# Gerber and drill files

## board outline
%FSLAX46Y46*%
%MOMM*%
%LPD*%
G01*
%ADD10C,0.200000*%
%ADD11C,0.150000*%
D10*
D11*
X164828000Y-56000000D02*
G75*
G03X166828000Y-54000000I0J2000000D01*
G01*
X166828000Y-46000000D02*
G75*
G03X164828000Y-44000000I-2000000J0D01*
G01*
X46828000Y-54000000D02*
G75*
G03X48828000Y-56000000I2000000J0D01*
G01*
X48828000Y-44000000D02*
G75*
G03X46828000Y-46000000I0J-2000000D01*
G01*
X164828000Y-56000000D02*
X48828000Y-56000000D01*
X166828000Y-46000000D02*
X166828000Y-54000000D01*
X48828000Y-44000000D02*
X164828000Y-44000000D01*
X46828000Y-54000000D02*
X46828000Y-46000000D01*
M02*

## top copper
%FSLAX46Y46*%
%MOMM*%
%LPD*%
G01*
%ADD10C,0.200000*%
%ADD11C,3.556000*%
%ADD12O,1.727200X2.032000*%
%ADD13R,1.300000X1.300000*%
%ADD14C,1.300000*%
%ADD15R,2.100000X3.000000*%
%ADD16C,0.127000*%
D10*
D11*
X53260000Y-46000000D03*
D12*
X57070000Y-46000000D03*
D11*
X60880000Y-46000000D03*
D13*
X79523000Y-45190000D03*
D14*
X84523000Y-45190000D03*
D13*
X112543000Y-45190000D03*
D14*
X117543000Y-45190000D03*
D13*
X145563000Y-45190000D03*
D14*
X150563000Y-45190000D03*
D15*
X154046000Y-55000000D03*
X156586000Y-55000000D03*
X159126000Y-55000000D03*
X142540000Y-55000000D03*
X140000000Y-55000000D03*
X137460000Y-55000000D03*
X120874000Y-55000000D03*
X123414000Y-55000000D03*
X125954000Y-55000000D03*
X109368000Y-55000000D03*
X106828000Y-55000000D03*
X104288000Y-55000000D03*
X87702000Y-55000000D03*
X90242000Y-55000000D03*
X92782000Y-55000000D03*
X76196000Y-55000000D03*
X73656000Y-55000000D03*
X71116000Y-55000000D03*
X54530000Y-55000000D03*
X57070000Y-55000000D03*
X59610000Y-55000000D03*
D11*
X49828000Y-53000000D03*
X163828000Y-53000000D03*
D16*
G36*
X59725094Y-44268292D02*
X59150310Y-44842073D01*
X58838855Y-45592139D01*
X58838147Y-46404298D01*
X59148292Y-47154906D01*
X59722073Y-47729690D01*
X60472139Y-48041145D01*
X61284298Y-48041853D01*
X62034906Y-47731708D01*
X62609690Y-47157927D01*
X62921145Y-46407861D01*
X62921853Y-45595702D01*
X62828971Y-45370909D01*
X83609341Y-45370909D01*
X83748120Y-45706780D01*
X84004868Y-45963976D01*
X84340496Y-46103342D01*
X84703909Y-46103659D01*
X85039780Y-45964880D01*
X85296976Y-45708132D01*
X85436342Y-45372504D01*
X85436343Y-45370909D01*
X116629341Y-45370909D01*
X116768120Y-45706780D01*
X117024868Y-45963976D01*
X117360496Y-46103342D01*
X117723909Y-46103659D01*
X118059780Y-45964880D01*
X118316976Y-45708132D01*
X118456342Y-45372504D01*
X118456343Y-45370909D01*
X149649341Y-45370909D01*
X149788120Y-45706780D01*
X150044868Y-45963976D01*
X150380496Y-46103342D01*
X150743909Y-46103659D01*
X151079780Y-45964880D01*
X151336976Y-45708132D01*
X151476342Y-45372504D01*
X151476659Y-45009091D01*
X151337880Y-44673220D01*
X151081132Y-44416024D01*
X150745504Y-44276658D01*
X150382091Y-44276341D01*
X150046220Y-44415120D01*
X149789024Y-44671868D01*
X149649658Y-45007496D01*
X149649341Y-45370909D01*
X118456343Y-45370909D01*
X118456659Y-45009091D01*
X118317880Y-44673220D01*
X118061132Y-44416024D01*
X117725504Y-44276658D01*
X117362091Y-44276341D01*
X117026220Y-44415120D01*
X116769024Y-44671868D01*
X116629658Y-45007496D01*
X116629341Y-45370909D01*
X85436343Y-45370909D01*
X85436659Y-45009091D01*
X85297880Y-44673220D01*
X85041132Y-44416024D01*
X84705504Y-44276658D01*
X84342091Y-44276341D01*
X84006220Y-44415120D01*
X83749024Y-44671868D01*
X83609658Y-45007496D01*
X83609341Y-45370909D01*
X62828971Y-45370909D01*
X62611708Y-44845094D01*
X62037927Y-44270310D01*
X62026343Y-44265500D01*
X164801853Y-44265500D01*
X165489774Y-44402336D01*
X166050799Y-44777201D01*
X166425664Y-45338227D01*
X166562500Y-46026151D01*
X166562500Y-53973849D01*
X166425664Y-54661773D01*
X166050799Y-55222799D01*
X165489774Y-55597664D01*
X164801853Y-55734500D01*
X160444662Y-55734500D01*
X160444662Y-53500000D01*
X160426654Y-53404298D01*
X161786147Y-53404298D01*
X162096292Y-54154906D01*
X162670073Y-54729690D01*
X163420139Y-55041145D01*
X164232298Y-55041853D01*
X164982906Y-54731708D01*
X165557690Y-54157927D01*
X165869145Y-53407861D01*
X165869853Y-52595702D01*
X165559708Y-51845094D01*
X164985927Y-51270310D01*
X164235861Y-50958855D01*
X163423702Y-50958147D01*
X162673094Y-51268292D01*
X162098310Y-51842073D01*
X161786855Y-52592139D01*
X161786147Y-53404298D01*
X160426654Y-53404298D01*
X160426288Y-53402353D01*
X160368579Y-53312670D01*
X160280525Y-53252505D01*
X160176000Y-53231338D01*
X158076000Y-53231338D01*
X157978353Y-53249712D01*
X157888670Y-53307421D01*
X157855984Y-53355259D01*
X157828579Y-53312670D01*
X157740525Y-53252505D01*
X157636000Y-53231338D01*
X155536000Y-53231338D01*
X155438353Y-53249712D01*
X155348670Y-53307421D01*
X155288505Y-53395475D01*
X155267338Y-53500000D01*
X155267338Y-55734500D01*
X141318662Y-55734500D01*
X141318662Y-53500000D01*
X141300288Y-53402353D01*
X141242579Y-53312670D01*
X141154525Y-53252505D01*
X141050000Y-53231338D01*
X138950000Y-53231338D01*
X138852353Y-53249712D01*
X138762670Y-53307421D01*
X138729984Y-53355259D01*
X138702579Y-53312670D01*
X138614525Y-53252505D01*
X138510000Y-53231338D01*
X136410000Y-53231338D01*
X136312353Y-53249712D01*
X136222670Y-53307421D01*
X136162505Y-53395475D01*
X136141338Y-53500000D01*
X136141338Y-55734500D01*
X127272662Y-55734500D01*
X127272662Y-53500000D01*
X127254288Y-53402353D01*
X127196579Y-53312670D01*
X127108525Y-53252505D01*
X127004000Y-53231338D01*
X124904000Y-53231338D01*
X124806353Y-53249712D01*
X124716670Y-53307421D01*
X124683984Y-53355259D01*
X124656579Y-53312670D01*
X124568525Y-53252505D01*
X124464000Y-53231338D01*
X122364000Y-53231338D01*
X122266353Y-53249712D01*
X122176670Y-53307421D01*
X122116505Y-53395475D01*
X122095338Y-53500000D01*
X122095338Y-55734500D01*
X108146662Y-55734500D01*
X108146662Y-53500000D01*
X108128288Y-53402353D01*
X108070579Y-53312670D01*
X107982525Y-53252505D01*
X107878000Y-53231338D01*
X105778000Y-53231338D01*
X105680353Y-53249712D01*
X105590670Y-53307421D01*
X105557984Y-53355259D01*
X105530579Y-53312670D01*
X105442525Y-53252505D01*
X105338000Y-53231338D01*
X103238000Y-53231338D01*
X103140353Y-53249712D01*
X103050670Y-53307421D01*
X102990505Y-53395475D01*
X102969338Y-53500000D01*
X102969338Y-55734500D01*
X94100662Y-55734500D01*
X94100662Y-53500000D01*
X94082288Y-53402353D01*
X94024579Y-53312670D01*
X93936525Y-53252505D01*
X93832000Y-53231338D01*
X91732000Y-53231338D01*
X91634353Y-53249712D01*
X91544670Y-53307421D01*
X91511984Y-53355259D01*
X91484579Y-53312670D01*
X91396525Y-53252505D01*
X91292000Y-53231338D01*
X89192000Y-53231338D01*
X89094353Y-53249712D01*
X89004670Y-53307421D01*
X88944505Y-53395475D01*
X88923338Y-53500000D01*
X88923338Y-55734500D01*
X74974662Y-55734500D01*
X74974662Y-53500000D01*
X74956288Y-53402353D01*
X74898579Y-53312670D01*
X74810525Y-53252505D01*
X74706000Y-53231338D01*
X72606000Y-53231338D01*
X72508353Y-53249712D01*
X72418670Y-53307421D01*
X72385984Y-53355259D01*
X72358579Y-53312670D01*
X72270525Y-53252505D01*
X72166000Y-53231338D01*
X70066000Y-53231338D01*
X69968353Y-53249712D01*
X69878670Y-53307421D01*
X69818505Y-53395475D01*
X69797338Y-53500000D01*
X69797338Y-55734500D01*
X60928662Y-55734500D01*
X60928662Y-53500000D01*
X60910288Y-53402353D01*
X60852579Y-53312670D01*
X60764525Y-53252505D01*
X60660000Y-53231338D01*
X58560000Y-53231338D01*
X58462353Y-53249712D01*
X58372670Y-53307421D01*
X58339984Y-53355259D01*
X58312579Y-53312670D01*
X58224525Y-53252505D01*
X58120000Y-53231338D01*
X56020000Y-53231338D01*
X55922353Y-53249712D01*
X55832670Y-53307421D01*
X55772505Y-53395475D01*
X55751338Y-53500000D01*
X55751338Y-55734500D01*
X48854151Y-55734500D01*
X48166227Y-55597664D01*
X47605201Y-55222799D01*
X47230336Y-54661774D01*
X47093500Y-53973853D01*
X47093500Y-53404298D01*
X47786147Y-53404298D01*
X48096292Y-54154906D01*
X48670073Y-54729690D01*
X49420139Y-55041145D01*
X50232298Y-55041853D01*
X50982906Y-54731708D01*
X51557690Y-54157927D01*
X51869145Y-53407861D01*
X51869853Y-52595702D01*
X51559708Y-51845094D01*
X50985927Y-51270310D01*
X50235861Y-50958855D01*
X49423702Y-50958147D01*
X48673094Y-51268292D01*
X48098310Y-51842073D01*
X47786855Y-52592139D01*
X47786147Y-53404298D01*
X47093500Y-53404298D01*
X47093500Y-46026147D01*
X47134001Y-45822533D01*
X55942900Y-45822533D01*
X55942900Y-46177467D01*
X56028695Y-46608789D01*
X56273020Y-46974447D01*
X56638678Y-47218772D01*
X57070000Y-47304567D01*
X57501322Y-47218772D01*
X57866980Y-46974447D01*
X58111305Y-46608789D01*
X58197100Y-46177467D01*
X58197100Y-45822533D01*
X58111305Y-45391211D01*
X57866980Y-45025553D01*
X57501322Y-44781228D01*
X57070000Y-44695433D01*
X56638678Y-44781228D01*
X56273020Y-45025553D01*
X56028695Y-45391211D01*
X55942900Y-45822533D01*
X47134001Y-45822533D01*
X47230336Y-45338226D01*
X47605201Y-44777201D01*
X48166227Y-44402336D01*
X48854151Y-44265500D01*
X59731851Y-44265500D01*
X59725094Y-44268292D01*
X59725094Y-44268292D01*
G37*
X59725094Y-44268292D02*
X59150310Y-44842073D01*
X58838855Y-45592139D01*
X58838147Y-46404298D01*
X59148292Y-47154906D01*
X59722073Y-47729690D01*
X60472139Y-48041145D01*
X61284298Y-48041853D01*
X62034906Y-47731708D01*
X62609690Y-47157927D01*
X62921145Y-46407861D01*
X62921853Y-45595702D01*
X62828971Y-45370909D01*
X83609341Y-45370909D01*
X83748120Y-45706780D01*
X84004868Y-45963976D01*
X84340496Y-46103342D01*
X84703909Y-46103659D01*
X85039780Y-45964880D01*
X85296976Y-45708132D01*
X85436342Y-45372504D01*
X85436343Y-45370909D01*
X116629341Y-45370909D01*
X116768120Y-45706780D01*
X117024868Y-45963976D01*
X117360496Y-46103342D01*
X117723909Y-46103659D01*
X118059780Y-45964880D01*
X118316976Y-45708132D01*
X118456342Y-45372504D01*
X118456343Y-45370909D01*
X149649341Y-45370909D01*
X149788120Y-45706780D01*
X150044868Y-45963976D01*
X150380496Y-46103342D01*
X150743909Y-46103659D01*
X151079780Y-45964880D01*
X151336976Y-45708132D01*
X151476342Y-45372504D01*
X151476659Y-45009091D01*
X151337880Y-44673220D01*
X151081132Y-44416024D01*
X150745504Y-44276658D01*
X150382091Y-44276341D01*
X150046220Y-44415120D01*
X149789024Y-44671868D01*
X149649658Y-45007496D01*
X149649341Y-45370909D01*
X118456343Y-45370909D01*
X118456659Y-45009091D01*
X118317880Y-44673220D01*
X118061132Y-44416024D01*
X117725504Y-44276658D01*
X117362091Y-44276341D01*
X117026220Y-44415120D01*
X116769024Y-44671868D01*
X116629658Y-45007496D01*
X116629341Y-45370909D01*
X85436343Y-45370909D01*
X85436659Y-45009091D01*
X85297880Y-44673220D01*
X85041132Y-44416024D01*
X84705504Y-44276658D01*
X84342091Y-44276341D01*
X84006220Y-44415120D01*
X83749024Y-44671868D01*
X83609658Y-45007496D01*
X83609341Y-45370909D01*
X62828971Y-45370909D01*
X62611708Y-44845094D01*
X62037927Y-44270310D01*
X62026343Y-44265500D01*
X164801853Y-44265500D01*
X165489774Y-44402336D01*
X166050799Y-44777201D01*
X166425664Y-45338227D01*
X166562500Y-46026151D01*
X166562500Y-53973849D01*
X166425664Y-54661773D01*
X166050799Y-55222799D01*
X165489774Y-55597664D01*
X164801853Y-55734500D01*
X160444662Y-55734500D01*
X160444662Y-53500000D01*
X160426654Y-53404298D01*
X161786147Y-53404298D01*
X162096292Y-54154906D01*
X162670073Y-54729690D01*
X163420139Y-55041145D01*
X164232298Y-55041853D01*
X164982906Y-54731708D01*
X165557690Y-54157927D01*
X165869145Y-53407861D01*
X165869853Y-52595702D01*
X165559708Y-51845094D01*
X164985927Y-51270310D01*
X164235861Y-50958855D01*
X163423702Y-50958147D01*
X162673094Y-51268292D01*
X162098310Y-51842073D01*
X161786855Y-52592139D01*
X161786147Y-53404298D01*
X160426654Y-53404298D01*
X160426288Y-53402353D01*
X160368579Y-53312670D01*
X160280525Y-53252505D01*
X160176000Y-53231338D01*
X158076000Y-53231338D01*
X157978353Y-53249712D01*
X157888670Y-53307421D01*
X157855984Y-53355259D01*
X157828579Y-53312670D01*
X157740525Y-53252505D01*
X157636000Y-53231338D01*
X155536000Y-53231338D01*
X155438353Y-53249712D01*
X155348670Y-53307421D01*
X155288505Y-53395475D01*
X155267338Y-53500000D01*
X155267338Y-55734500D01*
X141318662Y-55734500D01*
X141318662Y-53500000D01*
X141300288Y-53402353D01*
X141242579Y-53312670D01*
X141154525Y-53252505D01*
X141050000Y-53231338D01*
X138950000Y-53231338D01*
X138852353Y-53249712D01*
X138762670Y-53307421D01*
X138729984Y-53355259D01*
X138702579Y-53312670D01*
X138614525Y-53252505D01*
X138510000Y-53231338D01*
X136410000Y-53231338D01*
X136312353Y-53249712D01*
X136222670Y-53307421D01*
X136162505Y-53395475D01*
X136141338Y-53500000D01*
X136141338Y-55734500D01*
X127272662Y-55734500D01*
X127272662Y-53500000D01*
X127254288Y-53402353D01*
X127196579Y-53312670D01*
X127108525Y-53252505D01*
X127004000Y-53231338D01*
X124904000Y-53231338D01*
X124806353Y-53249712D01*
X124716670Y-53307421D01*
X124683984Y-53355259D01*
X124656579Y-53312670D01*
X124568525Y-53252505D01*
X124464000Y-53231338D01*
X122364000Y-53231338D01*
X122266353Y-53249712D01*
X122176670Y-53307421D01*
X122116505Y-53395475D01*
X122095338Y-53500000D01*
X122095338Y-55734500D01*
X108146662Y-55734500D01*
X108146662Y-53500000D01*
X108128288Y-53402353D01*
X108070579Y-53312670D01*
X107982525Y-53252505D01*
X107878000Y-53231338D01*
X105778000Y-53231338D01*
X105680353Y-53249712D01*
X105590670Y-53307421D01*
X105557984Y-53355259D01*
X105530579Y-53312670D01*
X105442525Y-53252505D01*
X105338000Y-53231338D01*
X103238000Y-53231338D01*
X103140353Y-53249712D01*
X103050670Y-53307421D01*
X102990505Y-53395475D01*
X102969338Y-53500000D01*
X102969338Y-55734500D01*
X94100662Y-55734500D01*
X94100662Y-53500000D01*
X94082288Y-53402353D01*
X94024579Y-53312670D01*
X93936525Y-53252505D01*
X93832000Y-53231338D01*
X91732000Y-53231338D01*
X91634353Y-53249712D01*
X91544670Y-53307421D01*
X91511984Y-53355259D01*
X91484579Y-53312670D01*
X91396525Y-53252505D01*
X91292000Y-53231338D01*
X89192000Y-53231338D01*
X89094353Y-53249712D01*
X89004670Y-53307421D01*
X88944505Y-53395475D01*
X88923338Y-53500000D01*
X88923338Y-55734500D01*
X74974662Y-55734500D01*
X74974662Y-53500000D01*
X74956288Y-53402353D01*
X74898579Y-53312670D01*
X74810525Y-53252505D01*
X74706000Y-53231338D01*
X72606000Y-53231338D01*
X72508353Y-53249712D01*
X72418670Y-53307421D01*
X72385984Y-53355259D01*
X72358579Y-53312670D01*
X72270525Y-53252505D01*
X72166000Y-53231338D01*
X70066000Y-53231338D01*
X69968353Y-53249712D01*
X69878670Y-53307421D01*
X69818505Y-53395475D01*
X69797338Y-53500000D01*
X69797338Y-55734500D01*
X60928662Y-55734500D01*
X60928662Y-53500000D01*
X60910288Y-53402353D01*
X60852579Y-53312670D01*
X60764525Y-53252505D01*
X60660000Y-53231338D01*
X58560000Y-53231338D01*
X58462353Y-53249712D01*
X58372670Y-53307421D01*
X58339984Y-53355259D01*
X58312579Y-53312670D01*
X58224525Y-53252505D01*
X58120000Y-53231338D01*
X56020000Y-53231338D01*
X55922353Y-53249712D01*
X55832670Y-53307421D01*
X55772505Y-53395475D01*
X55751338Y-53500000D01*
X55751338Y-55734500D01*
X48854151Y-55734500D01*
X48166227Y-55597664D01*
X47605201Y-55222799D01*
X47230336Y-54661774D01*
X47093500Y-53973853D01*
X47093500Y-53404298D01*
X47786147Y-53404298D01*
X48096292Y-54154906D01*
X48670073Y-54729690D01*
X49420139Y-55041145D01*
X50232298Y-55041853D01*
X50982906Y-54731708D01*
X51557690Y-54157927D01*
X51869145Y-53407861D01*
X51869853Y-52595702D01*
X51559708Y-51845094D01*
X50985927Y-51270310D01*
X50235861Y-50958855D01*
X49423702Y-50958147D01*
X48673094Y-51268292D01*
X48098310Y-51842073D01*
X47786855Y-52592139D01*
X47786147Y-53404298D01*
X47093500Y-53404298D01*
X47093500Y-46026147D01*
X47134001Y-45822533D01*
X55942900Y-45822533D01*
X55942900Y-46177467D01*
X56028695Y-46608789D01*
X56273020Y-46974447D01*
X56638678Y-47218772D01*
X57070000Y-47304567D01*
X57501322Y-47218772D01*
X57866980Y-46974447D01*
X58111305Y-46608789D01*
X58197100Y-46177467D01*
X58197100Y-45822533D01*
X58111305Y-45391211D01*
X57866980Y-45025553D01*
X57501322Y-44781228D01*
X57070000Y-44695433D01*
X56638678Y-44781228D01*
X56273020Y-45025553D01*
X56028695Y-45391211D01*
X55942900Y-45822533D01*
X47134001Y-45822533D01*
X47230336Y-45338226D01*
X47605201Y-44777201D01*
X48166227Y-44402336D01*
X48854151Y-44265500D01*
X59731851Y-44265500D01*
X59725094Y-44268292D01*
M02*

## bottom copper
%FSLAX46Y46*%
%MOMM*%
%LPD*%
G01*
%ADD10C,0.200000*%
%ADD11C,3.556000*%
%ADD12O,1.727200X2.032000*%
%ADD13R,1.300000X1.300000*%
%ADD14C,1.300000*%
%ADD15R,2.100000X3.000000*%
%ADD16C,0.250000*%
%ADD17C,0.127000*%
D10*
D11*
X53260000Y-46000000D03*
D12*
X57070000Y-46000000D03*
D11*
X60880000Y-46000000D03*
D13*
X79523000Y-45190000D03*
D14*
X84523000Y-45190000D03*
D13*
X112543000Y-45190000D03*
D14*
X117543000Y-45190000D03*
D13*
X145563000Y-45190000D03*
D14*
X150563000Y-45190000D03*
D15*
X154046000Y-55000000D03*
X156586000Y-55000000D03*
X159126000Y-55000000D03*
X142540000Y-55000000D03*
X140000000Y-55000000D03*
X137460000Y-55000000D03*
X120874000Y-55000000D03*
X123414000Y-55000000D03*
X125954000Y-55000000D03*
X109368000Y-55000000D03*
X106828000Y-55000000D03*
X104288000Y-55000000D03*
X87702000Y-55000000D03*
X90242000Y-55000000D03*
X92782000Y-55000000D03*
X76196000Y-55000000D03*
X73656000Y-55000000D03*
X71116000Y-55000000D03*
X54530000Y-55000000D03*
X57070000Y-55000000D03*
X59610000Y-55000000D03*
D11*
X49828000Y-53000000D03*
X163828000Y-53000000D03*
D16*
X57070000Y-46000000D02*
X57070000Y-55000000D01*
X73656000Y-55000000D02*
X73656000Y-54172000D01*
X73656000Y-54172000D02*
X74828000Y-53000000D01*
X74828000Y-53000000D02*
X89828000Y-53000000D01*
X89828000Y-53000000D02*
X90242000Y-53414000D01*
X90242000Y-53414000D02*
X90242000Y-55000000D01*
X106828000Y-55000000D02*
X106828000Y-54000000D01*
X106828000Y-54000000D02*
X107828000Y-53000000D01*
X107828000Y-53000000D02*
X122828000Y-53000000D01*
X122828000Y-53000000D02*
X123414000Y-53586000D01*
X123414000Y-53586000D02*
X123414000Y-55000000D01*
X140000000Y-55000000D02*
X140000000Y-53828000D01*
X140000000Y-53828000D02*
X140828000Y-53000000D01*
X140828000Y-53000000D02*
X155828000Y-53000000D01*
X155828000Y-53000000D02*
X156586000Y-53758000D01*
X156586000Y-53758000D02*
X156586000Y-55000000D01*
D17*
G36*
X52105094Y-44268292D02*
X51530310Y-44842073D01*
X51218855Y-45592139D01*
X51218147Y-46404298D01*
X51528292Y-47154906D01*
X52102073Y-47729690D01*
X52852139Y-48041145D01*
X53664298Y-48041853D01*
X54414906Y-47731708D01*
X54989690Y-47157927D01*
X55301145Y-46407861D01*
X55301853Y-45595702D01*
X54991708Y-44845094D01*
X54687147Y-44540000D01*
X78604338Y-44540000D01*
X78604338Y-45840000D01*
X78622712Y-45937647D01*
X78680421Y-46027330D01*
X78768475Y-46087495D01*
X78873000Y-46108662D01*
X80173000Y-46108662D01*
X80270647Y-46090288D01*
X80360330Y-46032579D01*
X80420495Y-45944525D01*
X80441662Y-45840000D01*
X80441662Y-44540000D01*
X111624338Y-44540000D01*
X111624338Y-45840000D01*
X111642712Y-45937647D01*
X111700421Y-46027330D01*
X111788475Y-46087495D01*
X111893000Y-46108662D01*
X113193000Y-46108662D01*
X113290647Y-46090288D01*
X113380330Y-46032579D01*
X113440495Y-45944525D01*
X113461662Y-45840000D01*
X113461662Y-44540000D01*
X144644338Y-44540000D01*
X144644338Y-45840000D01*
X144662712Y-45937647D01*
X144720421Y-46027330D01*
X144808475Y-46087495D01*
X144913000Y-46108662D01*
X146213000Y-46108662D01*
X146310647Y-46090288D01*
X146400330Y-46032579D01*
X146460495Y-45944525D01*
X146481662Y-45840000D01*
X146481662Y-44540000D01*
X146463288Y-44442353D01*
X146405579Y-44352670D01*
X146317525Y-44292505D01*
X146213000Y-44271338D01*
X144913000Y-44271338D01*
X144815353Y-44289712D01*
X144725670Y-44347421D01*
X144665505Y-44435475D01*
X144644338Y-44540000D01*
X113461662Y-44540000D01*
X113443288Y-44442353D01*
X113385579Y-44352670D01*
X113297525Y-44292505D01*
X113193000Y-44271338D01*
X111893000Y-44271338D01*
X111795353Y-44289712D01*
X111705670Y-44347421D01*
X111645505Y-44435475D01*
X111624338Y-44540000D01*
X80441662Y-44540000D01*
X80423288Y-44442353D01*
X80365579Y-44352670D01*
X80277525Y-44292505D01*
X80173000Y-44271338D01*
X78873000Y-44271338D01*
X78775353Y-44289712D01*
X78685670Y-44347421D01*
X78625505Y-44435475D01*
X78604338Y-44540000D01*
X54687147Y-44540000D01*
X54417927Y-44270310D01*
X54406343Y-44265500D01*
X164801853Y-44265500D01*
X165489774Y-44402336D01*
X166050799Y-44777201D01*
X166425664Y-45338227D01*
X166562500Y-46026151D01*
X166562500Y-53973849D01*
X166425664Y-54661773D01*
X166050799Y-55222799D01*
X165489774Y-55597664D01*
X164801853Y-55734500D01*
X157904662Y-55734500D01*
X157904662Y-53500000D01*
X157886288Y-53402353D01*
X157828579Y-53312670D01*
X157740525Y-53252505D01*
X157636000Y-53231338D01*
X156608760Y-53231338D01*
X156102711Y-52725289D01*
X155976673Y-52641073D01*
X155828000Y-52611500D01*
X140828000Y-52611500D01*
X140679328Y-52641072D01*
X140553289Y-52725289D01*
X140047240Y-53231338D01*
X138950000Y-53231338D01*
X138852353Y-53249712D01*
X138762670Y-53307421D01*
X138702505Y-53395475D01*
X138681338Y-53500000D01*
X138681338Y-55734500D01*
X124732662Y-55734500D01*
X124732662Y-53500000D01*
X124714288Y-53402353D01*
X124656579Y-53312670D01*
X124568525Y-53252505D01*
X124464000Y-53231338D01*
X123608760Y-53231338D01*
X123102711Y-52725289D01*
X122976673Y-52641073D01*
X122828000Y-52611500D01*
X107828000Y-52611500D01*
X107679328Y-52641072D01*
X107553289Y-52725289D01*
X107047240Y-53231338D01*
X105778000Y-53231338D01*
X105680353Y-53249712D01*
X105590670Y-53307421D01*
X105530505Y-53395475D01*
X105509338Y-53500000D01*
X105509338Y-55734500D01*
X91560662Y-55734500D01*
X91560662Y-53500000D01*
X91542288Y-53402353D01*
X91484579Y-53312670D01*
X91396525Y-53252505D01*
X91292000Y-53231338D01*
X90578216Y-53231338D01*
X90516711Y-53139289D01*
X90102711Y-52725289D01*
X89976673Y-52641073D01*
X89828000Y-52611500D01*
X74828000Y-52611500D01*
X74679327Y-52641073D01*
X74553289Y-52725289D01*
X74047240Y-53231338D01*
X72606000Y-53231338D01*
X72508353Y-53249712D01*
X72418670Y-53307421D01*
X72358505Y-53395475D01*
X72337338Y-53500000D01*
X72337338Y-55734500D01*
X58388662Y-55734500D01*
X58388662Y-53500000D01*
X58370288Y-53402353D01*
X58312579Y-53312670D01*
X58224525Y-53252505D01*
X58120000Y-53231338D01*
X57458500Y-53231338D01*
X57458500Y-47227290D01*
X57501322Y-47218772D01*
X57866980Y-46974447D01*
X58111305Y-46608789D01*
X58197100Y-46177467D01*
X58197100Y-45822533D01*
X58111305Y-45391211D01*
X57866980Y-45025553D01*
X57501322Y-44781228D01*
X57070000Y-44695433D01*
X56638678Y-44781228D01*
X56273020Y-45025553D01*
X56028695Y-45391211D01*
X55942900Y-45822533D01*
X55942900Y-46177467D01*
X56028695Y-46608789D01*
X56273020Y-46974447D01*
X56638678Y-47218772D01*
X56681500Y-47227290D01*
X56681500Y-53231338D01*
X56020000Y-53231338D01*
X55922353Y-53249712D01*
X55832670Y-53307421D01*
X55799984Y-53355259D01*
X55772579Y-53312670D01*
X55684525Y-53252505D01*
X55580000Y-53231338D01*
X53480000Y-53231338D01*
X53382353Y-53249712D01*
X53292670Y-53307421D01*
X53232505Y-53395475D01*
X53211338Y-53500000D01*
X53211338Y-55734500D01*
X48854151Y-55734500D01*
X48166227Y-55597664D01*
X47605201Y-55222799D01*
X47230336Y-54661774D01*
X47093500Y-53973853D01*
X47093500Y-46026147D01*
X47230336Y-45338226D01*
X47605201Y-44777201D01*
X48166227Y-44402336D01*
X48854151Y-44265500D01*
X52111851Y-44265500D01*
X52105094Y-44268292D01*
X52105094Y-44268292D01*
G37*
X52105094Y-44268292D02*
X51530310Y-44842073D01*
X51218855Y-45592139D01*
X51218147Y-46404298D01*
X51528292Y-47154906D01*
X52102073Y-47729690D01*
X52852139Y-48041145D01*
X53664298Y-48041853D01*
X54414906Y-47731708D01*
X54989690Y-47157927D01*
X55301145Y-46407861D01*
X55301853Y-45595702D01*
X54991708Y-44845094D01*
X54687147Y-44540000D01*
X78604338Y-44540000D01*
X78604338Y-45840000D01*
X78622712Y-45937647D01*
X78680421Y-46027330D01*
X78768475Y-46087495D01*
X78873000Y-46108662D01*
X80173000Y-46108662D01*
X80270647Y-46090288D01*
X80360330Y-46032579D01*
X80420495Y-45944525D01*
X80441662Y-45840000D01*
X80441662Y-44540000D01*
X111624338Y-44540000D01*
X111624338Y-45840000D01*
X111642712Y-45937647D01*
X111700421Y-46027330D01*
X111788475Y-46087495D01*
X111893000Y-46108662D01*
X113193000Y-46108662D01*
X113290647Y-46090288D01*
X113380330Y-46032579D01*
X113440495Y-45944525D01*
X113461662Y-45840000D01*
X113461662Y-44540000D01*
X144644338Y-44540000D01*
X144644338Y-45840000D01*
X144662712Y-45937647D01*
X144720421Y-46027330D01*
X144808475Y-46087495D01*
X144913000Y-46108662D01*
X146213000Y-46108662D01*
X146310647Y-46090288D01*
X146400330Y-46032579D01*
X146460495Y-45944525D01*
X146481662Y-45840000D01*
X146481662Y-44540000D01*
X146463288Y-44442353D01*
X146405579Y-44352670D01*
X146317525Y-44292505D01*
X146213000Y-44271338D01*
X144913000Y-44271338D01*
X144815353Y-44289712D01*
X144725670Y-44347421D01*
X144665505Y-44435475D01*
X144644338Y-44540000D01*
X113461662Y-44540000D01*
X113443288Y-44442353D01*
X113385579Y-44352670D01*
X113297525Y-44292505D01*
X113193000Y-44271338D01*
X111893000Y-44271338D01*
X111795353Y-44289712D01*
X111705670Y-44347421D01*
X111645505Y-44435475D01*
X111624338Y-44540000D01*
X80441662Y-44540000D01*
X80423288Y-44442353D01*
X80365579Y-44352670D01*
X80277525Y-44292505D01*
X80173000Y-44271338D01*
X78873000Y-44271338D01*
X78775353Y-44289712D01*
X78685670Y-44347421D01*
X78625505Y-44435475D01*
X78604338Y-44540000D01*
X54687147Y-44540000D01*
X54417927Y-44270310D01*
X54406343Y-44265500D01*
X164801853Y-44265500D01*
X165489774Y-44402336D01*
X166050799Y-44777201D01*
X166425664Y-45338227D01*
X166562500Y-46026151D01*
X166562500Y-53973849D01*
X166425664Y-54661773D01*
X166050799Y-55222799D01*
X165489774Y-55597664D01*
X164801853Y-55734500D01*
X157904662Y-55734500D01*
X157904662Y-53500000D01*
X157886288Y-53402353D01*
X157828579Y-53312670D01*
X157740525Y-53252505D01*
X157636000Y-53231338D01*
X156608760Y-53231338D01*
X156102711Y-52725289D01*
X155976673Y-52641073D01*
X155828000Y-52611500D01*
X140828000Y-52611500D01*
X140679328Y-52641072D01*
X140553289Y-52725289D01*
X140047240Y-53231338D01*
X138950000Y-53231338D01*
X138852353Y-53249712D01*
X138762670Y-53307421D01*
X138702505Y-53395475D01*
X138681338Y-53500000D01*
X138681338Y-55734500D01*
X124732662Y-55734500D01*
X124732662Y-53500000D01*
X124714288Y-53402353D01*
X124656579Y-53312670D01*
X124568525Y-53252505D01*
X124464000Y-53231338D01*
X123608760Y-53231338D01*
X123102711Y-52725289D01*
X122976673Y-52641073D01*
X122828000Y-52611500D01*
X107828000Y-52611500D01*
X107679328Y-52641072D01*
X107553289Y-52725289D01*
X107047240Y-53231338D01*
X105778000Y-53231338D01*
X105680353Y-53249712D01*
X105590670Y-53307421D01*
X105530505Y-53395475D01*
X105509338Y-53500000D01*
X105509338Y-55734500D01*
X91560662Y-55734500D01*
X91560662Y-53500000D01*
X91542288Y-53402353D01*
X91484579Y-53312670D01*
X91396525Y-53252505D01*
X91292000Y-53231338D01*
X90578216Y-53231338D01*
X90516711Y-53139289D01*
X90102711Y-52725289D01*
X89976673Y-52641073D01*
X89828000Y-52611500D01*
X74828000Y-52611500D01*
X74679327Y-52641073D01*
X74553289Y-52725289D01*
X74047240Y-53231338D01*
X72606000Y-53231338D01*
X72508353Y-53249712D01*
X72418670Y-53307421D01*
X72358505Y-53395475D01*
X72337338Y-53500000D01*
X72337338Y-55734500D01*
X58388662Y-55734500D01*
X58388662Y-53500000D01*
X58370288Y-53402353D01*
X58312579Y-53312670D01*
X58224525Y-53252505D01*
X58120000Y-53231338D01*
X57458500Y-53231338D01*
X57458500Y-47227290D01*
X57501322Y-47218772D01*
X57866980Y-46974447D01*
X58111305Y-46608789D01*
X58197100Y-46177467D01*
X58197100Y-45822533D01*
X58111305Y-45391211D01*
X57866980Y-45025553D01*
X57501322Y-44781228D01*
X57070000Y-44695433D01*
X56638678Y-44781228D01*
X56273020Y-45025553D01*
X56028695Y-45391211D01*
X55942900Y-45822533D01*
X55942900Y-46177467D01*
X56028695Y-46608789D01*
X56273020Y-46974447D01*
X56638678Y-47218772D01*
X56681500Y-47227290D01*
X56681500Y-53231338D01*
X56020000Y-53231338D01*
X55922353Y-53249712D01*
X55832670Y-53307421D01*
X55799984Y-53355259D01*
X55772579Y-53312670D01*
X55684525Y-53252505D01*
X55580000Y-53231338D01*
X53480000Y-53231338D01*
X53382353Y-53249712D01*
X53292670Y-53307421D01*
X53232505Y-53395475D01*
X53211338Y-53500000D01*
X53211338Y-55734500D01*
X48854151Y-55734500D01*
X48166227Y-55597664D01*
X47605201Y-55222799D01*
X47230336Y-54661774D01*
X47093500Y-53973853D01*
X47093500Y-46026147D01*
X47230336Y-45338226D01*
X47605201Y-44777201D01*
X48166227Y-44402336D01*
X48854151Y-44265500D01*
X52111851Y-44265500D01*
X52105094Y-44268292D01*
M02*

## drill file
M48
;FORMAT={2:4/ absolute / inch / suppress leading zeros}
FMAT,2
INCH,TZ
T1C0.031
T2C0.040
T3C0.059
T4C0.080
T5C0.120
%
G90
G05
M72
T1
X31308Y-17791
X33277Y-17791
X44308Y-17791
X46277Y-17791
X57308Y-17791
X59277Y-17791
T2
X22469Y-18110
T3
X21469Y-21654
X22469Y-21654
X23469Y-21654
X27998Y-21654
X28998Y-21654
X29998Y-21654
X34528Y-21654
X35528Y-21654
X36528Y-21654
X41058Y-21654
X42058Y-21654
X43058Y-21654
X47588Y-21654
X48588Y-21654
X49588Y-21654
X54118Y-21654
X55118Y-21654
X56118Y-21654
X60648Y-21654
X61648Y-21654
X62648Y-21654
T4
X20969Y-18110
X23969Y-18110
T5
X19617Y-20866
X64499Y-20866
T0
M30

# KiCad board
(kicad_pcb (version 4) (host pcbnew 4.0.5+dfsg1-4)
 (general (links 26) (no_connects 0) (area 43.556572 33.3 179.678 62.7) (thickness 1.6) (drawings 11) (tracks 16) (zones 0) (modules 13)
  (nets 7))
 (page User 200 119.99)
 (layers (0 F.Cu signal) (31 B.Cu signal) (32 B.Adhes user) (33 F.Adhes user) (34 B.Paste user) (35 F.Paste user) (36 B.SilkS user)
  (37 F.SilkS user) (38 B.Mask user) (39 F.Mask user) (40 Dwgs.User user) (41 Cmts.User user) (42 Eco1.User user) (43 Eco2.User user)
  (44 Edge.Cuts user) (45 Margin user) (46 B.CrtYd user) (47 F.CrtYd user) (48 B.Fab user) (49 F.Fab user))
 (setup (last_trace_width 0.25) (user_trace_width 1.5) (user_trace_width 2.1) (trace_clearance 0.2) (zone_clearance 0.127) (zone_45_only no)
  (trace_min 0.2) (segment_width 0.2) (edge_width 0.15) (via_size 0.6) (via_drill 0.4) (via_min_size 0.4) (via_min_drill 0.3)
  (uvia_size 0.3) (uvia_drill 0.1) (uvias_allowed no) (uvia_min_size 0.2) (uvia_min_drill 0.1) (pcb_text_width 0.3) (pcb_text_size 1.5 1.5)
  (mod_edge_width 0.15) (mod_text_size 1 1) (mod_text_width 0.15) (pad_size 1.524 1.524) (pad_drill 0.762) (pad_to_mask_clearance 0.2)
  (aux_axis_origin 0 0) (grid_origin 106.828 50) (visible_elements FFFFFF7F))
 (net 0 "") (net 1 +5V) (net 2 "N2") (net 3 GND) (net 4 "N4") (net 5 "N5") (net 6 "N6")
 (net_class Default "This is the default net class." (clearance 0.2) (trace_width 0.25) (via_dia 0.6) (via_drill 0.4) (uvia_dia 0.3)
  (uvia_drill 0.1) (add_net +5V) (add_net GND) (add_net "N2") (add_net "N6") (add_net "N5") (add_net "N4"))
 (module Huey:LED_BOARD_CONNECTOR (layer F.Cu) (at 57.07 46 90)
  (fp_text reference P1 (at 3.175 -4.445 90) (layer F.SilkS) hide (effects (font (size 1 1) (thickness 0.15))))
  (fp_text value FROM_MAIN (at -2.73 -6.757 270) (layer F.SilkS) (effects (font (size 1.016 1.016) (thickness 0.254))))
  (pad 1 thru_hole circle (at 0 -3.81 90) (size 3.556 3.556) (drill 2.032) (layers *.Cu *.Mask) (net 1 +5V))
  (pad 2 thru_hole oval (at 0 0 90) (size 2.032 1.7272) (drill 1.016) (layers *.Cu *.Mask) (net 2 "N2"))
  (pad 3 thru_hole circle (at 0 3.81 90) (size 3.556 3.556) (drill 2.032) (layers *.Cu *.Mask) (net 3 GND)))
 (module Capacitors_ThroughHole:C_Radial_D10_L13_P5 (layer F.Cu) (at 79.523 45.19)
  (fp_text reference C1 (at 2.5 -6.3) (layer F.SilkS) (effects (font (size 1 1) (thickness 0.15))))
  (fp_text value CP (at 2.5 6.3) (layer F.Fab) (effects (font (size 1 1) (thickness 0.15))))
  (pad 1 thru_hole rect (at 0 0) (size 1.3 1.3) (drill 0.8) (layers *.Cu *.Mask) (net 1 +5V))
  (pad 2 thru_hole circle (at 5 0) (size 1.3 1.3) (drill 0.8) (layers *.Cu *.Mask) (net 3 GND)))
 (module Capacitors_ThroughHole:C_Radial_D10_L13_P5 (layer F.Cu) (at 112.543 45.19)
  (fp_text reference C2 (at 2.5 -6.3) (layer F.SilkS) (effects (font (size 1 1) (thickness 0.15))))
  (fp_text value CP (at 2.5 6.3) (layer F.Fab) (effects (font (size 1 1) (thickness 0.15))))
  (pad 1 thru_hole rect (at 0 0) (size 1.3 1.3) (drill 0.8) (layers *.Cu *.Mask) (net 1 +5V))
  (pad 2 thru_hole circle (at 5 0) (size 1.3 1.3) (drill 0.8) (layers *.Cu *.Mask) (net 3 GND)))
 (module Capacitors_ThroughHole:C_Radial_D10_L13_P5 (layer F.Cu) (at 145.563 45.19)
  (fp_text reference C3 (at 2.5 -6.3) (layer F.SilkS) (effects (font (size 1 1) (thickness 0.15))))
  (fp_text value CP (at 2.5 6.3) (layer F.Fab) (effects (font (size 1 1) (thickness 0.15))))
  (pad 1 thru_hole rect (at 0 0) (size 1.3 1.3) (drill 0.8) (layers *.Cu *.Mask) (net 1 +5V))
  (pad 2 thru_hole circle (at 5 0) (size 1.3 1.3) (drill 0.8) (layers *.Cu *.Mask) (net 3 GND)))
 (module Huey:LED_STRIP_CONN (layer F.Cu) (at 156.586 55 90)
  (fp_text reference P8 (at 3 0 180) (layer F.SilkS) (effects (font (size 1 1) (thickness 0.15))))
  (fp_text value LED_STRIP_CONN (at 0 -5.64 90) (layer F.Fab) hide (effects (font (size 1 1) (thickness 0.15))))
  (pad 1 thru_hole rect (at 0 -2.54 90) (size 3 2.1) (drill 1.5) (layers *.Cu *.Mask) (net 1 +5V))
  (pad 2 thru_hole rect (at 0 0 90) (size 3 2.1) (drill 1.5) (layers *.Cu *.Mask) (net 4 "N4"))
  (pad 3 thru_hole rect (at 0 2.54 90) (size 3 2.1) (drill 1.5) (layers *.Cu *.Mask) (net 3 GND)))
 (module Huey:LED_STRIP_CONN (layer F.Cu) (at 140 55 270)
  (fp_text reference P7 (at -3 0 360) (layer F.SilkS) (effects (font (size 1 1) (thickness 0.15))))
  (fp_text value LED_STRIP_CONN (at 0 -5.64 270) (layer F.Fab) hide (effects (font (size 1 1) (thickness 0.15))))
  (pad 1 thru_hole rect (at 0 -2.54 270) (size 3 2.1) (drill 1.5) (layers *.Cu *.Mask) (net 1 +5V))
  (pad 2 thru_hole rect (at 0 0 270) (size 3 2.1) (drill 1.5) (layers *.Cu *.Mask) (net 4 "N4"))
  (pad 3 thru_hole rect (at 0 2.54 270) (size 3 2.1) (drill 1.5) (layers *.Cu *.Mask) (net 3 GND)))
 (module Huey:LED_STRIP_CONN (layer F.Cu) (at 123.414 55 90)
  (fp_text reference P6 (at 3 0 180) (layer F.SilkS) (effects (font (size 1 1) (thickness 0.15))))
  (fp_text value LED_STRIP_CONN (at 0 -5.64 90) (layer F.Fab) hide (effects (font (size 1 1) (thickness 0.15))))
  (pad 1 thru_hole rect (at 0 -2.54 90) (size 3 2.1) (drill 1.5) (layers *.Cu *.Mask) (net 1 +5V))
  (pad 2 thru_hole rect (at 0 0 90) (size 3 2.1) (drill 1.5) (layers *.Cu *.Mask) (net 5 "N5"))
  (pad 3 thru_hole rect (at 0 2.54 90) (size 3 2.1) (drill 1.5) (layers *.Cu *.Mask) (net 3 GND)))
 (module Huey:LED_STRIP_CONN (layer F.Cu) (at 106.828 55 270)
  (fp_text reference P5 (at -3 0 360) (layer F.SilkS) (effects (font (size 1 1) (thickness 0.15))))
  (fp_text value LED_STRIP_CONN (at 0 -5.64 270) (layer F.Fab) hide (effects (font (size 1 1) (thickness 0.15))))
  (pad 1 thru_hole rect (at 0 -2.54 270) (size 3 2.1) (drill 1.5) (layers *.Cu *.Mask) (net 1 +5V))
  (pad 2 thru_hole rect (at 0 0 270) (size 3 2.1) (drill 1.5) (layers *.Cu *.Mask) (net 5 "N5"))
  (pad 3 thru_hole rect (at 0 2.54 270) (size 3 2.1) (drill 1.5) (layers *.Cu *.Mask) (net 3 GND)))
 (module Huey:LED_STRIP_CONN (layer F.Cu) (at 90.242 55 90)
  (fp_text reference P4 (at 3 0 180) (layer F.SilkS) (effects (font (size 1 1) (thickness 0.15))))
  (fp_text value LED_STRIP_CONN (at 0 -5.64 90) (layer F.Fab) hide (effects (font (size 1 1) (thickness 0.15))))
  (pad 1 thru_hole rect (at 0 -2.54 90) (size 3 2.1) (drill 1.5) (layers *.Cu *.Mask) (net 1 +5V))
  (pad 2 thru_hole rect (at 0 0 90) (size 3 2.1) (drill 1.5) (layers *.Cu *.Mask) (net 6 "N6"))
  (pad 3 thru_hole rect (at 0 2.54 90) (size 3 2.1) (drill 1.5) (layers *.Cu *.Mask) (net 3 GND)))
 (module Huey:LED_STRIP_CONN (layer F.Cu) (at 73.656 55 270)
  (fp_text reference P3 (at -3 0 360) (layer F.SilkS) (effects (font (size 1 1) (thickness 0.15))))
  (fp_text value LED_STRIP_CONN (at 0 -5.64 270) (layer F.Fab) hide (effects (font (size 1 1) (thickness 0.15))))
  (pad 1 thru_hole rect (at 0 -2.54 270) (size 3 2.1) (drill 1.5) (layers *.Cu *.Mask) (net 1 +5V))
  (pad 2 thru_hole rect (at 0 0 270) (size 3 2.1) (drill 1.5) (layers *.Cu *.Mask) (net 6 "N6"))
  (pad 3 thru_hole rect (at 0 2.54 270) (size 3 2.1) (drill 1.5) (layers *.Cu *.Mask) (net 3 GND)))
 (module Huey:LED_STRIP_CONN (layer F.Cu) (at 57.07 55 90)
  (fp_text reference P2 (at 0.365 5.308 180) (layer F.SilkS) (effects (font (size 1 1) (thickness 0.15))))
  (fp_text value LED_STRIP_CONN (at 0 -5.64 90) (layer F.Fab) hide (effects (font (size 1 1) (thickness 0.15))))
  (pad 1 thru_hole rect (at 0 -2.54 90) (size 3 2.1) (drill 1.5) (layers *.Cu *.Mask) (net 1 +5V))
  (pad 2 thru_hole rect (at 0 0 90) (size 3 2.1) (drill 1.5) (layers *.Cu *.Mask) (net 2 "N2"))
  (pad 3 thru_hole rect (at 0 2.54 90) (size 3 2.1) (drill 1.5) (layers *.Cu *.Mask) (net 3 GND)))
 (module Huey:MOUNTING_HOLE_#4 (layer F.Cu) (at 49.828 53)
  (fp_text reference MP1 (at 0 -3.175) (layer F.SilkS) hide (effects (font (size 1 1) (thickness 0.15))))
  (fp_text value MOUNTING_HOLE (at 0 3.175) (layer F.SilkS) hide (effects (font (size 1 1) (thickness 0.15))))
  (pad 1 thru_hole circle (at 0 0) (size 3.556 3.556) (drill 3.048) (layers *.Cu *.Mask F.SilkS) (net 3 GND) (zone_connect 2)))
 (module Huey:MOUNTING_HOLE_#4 (layer F.Cu) (at 163.828 53)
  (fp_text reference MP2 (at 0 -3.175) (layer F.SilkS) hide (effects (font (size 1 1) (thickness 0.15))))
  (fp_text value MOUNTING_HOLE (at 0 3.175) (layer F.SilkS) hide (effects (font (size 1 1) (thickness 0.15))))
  (pad 1 thru_hole circle (at 0 0) (size 3.556 3.556) (drill 3.048) (layers *.Cu *.Mask F.SilkS) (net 3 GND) (zone_connect 2)))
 (gr_arc (start 164.828 54) (end 166.828 54) (angle 90) (layer Edge.Cuts) (width 0.15))
 (gr_arc (start 164.828 46) (end 164.828 44) (angle 90) (layer Edge.Cuts) (width 0.15))
 (gr_arc (start 48.828 54) (end 48.828 56) (angle 90) (layer Edge.Cuts) (width 0.15))
 (gr_arc (start 48.828 46) (end 46.828 46) (angle 90) (layer Edge.Cuts) (width 0.15))
 (gr_line (start 164.828 56) (end 48.828 56) (layer Edge.Cuts) (width 0.15))
 (gr_line (start 166.828 46) (end 166.828 54) (angle 90) (layer Edge.Cuts) (width 0.15))
 (gr_line (start 48.828 44) (end 164.828 44) (angle 90) (layer Edge.Cuts) (width 0.15))
 (gr_line (start 46.828 54) (end 46.828 46) (angle 90) (layer Edge.Cuts) (width 0.15))
 (segment (start 57.07 46) (end 57.07 55) (width 0.25) (layer B.Cu) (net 2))
 (segment (start 73.656 55) (end 73.656 54.172) (width 0.25) (layer B.Cu) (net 6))
 (segment (start 73.656 54.172) (end 74.828 53) (width 0.25) (layer B.Cu) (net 6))
 (segment (start 74.828 53) (end 89.828 53) (width 0.25) (layer B.Cu) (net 6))
 (segment (start 89.828 53) (end 90.242 53.414) (width 0.25) (layer B.Cu) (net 6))
 (segment (start 90.242 53.414) (end 90.242 55) (width 0.25) (layer B.Cu) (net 6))
 (segment (start 106.828 55) (end 106.828 54) (width 0.25) (layer B.Cu) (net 5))
 (segment (start 106.828 54) (end 107.828 53) (width 0.25) (layer B.Cu) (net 5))
 (segment (start 107.828 53) (end 122.828 53) (width 0.25) (layer B.Cu) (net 5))
 (segment (start 122.828 53) (end 123.414 53.586) (width 0.25) (layer B.Cu) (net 5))
 (segment (start 123.414 53.586) (end 123.414 55) (width 0.25) (layer B.Cu) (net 5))
 (segment (start 140 55) (end 140 53.828) (width 0.25) (layer B.Cu) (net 4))
 (segment (start 140 53.828) (end 140.828 53) (width 0.25) (layer B.Cu) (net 4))
 (segment (start 140.828 53) (end 155.828 53) (width 0.25) (layer B.Cu) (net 4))
 (segment (start 155.828 53) (end 156.586 53.758) (width 0.25) (layer B.Cu) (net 4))
 (segment (start 156.586 53.758) (end 156.586 55) (width 0.25) (layer B.Cu) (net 4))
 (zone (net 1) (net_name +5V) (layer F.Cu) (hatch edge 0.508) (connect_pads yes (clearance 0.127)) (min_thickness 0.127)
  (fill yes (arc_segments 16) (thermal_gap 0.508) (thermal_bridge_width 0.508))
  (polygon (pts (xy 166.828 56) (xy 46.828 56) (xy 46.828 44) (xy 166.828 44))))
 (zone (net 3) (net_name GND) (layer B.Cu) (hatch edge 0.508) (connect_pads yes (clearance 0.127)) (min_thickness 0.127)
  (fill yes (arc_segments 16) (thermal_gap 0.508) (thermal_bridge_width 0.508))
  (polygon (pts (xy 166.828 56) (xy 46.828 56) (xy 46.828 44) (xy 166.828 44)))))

